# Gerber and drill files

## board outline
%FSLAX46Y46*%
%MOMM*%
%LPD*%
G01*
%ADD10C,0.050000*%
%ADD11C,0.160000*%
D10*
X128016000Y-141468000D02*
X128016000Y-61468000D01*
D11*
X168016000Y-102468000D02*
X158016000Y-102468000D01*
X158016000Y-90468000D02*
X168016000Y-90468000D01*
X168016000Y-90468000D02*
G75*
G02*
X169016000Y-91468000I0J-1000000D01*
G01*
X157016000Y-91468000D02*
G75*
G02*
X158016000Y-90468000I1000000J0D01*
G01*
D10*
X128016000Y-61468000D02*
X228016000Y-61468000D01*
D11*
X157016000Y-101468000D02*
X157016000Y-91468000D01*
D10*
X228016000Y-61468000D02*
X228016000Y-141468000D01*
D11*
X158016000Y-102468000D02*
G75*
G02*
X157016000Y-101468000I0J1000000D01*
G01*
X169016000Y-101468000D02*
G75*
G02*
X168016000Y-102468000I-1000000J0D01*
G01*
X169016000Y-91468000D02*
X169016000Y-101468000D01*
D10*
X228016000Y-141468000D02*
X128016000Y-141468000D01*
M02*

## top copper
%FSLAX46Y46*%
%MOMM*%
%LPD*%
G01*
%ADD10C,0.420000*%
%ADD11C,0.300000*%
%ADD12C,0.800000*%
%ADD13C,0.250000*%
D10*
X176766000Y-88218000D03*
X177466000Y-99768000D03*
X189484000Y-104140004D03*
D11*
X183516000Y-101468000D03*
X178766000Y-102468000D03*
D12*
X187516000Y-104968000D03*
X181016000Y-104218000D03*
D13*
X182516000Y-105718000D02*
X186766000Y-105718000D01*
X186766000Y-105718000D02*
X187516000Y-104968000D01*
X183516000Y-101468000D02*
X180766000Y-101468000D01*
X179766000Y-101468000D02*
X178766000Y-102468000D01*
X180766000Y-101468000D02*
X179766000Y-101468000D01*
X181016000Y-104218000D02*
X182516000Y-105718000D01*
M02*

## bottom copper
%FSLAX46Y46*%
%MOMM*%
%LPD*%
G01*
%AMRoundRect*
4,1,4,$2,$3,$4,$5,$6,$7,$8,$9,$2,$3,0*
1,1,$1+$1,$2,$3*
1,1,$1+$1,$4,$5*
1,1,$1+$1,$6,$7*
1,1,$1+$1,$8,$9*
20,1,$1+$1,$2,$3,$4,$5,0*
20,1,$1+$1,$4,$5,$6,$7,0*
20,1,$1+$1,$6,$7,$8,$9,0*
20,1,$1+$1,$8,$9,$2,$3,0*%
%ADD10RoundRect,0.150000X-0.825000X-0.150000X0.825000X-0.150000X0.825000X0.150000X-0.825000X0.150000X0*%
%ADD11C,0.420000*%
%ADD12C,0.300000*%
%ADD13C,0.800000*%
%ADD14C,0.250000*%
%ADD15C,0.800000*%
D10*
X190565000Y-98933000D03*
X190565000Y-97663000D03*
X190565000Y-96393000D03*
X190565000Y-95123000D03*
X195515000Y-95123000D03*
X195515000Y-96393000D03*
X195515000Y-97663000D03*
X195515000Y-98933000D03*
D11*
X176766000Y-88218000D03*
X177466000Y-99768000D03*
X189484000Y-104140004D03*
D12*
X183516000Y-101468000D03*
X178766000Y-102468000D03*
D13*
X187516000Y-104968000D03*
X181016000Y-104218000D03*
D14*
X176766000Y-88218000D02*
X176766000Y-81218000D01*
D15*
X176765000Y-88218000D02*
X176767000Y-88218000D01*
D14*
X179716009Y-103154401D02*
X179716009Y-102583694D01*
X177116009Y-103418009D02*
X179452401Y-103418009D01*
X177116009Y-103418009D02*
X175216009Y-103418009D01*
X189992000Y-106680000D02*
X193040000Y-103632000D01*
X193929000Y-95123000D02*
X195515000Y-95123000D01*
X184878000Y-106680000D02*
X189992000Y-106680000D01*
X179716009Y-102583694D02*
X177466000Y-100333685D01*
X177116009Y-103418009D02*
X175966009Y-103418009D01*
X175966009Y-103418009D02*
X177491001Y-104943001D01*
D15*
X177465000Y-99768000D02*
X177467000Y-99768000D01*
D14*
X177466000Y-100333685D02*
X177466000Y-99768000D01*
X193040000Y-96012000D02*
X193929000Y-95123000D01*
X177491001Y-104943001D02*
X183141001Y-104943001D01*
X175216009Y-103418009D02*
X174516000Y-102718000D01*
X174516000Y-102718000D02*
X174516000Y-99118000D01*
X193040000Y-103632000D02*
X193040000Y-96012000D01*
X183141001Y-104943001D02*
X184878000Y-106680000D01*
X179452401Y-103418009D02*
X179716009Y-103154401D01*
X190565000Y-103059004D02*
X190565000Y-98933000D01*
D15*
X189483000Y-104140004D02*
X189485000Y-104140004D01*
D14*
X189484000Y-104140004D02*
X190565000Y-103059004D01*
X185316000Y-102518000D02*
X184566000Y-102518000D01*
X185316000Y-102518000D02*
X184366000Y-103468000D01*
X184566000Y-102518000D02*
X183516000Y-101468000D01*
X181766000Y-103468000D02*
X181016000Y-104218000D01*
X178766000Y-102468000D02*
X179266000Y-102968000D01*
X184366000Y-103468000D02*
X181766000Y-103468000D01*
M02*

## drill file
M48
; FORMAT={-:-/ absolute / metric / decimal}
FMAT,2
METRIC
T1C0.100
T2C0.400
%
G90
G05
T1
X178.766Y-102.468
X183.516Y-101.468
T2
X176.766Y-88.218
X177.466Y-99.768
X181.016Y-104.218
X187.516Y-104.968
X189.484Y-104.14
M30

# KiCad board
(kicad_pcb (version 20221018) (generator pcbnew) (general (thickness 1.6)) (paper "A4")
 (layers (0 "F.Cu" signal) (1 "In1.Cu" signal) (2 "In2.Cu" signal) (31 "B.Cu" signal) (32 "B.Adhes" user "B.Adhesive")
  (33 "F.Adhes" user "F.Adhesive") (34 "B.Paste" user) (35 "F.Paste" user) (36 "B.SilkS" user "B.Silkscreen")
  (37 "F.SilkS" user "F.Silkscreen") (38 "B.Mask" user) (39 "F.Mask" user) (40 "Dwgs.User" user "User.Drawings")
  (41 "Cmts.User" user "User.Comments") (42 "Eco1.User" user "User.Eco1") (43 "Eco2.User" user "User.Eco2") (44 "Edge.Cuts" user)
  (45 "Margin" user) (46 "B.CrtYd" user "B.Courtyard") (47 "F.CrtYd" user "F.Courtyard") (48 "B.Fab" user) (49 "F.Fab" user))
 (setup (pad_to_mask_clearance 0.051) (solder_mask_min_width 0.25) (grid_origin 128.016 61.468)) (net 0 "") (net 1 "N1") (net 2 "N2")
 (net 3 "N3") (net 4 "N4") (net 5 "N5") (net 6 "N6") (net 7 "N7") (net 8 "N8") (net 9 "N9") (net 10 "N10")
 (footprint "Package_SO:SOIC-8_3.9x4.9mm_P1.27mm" (layer "B.Cu") (at 193.04 97.028)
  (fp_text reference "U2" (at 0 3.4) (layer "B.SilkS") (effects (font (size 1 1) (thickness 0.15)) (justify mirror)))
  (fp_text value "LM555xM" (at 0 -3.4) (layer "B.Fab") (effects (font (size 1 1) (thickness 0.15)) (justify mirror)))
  (pad "1" smd roundrect (at -2.475 1.905) (size 1.95 0.6) (layers "B.Cu" "B.Paste" "B.Mask") (roundrect_rratio 0.25) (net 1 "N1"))
  (pad "2" smd roundrect (at -2.475 0.635) (size 1.95 0.6) (layers "B.Cu" "B.Paste" "B.Mask") (roundrect_rratio 0.25) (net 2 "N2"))
  (pad "3" smd roundrect (at -2.475 -0.635) (size 1.95 0.6) (layers "B.Cu" "B.Paste" "B.Mask") (roundrect_rratio 0.25) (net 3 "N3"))
  (pad "4" smd roundrect (at -2.475 -1.905) (size 1.95 0.6) (layers "B.Cu" "B.Paste" "B.Mask") (roundrect_rratio 0.25) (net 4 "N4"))
  (pad "5" smd roundrect (at 2.475 -1.905) (size 1.95 0.6) (layers "B.Cu" "B.Paste" "B.Mask") (roundrect_rratio 0.25) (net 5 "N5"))
  (pad "6" smd roundrect (at 2.475 -0.635) (size 1.95 0.6) (layers "B.Cu" "B.Paste" "B.Mask") (roundrect_rratio 0.25) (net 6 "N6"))
  (pad "7" smd roundrect (at 2.475 0.635) (size 1.95 0.6) (layers "B.Cu" "B.Paste" "B.Mask") (roundrect_rratio 0.25) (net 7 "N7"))
  (pad "8" smd roundrect (at 2.475 1.905) (size 1.95 0.6) (layers "B.Cu" "B.Paste" "B.Mask") (roundrect_rratio 0.25) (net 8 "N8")))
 (gr_line (start 128.016 141.468) (end 128.016 61.468) (stroke (width 0.05) (type solid)) (layer "Edge.Cuts"))
 (gr_line (start 168.016 102.468) (end 158.016 102.468) (stroke (width 0.16) (type solid)) (layer "Edge.Cuts"))
 (gr_line (start 158.016 90.468) (end 168.016 90.468) (stroke (width 0.16) (type solid)) (layer "Edge.Cuts"))
 (gr_arc (start 168.016 90.468) (mid 168.723107 90.760893) (end 169.016 91.468) (stroke (width 0.16) (type solid)) (layer "Edge.Cuts"))
 (gr_arc (start 157.016 91.468) (mid 157.308893 90.760893) (end 158.016 90.468) (stroke (width 0.16) (type solid)) (layer "Edge.Cuts"))
 (gr_line (start 128.016 61.468) (end 228.016 61.468) (stroke (width 0.05) (type solid)) (layer "Edge.Cuts"))
 (gr_line (start 157.016 101.468) (end 157.016 91.468) (stroke (width 0.16) (type solid)) (layer "Edge.Cuts"))
 (gr_line (start 228.016 61.468) (end 228.016 141.468) (stroke (width 0.05) (type solid)) (layer "Edge.Cuts"))
 (gr_arc (start 158.016 102.468) (mid 157.308893 102.175107) (end 157.016 101.468) (stroke (width 0.16) (type solid)) (layer "Edge.Cuts"))
 (gr_arc (start 169.016 101.468) (mid 168.723107 102.175107) (end 168.016 102.468) (stroke (width 0.16) (type solid)) (layer "Edge.Cuts"))
 (gr_line (start 169.016 91.468) (end 169.016 101.468) (stroke (width 0.16) (type solid)) (layer "Edge.Cuts"))
 (gr_line (start 228.016 141.468) (end 128.016 141.468) (stroke (width 0.05) (type solid)) (layer "Edge.Cuts"))
 (via (at 176.766 88.218) (size 0.42) (drill 0.4) (layers "F.Cu" "B.Cu") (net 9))
 (segment (start 176.766 88.218) (end 176.766 81.218) (width 0.25) (layer "B.Cu") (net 9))
 (segment (start 176.765 88.218) (end 176.767 88.218) (width 0.8) (layer "B.Cu") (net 9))
 (via (at 177.466 99.768) (size 0.42) (drill 0.4) (layers "F.Cu" "B.Cu") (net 5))
 (segment (start 179.716009 103.154401) (end 179.716009 102.583694) (width 0.25) (layer "B.Cu") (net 5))
 (segment (start 177.116009 103.418009) (end 179.452401 103.418009) (width 0.25) (layer "B.Cu") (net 5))
 (segment (start 177.116009 103.418009) (end 175.216009 103.418009) (width 0.25) (layer "B.Cu") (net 5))
 (segment (start 189.992 106.68) (end 193.04 103.632) (width 0.25) (layer "B.Cu") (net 5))
 (segment (start 193.929 95.123) (end 195.515 95.123) (width 0.25) (layer "B.Cu") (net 5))
 (segment (start 184.878 106.68) (end 189.992 106.68) (width 0.25) (layer "B.Cu") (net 5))
 (segment (start 179.716009 102.583694) (end 177.466 100.333685) (width 0.25) (layer "B.Cu") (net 5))
 (segment (start 177.116009 103.418009) (end 175.966009 103.418009) (width 0.25) (layer "B.Cu") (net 5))
 (segment (start 175.966009 103.418009) (end 177.491001 104.943001) (width 0.25) (layer "B.Cu") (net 5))
 (segment (start 177.465 99.768) (end 177.467 99.768) (width 0.8) (layer "B.Cu") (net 5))
 (segment (start 177.466 100.333685) (end 177.466 99.768) (width 0.25) (layer "B.Cu") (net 5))
 (segment (start 193.04 96.012) (end 193.929 95.123) (width 0.25) (layer "B.Cu") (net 5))
 (segment (start 177.491001 104.943001) (end 183.141001 104.943001) (width 0.25) (layer "B.Cu") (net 5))
 (segment (start 175.216009 103.418009) (end 174.516 102.718) (width 0.25) (layer "B.Cu") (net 5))
 (segment (start 174.516 102.718) (end 174.516 99.118) (width 0.25) (layer "B.Cu") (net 5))
 (segment (start 193.04 103.632) (end 193.04 96.012) (width 0.25) (layer "B.Cu") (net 5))
 (segment (start 183.141001 104.943001) (end 184.878 106.68) (width 0.25) (layer "B.Cu") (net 5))
 (segment (start 179.452401 103.418009) (end 179.716009 103.154401) (width 0.25) (layer "B.Cu") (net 5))
 (via (at 189.484 104.140004) (size 0.42) (drill 0.4) (layers "F.Cu" "B.Cu") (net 1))
 (segment (start 190.565 103.059004) (end 190.565 98.933) (width 0.25) (layer "B.Cu") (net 1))
 (segment (start 189.483 104.140004) (end 189.485 104.140004) (width 0.8) (layer "B.Cu") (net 1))
 (segment (start 189.484 104.140004) (end 190.565 103.059004) (width 0.25) (layer "B.Cu") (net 1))
 (segment (start 182.516 105.718) (end 186.766 105.718) (width 0.25) (layer "F.Cu") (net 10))
 (segment (start 186.766 105.718) (end 187.516 104.968) (width 0.25) (layer "F.Cu") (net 10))
 (segment (start 183.516 101.468) (end 180.766 101.468) (width 0.25) (layer "F.Cu") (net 10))
 (segment (start 179.766 101.468) (end 178.766 102.468) (width 0.25) (layer "F.Cu") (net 10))
 (segment (start 180.766 101.468) (end 179.766 101.468) (width 0.25) (layer "F.Cu") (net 10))
 (segment (start 181.016 104.218) (end 182.516 105.718) (width 0.25) (layer "F.Cu") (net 10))
 (segment (start 185.316 102.518) (end 184.566 102.518) (width 0.25) (layer "B.Cu") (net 10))
 (segment (start 185.316 102.518) (end 184.366 103.468) (width 0.25) (layer "B.Cu") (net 10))
 (segment (start 184.566 102.518) (end 183.516 101.468) (width 0.25) (layer "B.Cu") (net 10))
 (segment (start 181.766 103.468) (end 181.016 104.218) (width 0.25) (layer "B.Cu") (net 10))
 (segment (start 178.766 102.468) (end 179.266 102.968) (width 0.25) (layer "B.Cu") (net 10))
 (segment (start 184.366 103.468) (end 181.766 103.468) (width 0.25) (layer "B.Cu") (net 10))
 (via (at 183.516 101.468) (size 0.3) (drill 0.1) (layers "F.Cu" "B.Cu") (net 10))
 (via (at 178.766 102.468) (size 0.3) (drill 0.1) (layers "F.Cu" "B.Cu") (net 10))
 (via (at 187.516 104.968) (size 0.8) (drill 0.4) (layers "F.Cu" "B.Cu") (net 10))
 (via (at 181.016 104.218) (size 0.8) (drill 0.4) (layers "F.Cu" "B.Cu") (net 10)))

